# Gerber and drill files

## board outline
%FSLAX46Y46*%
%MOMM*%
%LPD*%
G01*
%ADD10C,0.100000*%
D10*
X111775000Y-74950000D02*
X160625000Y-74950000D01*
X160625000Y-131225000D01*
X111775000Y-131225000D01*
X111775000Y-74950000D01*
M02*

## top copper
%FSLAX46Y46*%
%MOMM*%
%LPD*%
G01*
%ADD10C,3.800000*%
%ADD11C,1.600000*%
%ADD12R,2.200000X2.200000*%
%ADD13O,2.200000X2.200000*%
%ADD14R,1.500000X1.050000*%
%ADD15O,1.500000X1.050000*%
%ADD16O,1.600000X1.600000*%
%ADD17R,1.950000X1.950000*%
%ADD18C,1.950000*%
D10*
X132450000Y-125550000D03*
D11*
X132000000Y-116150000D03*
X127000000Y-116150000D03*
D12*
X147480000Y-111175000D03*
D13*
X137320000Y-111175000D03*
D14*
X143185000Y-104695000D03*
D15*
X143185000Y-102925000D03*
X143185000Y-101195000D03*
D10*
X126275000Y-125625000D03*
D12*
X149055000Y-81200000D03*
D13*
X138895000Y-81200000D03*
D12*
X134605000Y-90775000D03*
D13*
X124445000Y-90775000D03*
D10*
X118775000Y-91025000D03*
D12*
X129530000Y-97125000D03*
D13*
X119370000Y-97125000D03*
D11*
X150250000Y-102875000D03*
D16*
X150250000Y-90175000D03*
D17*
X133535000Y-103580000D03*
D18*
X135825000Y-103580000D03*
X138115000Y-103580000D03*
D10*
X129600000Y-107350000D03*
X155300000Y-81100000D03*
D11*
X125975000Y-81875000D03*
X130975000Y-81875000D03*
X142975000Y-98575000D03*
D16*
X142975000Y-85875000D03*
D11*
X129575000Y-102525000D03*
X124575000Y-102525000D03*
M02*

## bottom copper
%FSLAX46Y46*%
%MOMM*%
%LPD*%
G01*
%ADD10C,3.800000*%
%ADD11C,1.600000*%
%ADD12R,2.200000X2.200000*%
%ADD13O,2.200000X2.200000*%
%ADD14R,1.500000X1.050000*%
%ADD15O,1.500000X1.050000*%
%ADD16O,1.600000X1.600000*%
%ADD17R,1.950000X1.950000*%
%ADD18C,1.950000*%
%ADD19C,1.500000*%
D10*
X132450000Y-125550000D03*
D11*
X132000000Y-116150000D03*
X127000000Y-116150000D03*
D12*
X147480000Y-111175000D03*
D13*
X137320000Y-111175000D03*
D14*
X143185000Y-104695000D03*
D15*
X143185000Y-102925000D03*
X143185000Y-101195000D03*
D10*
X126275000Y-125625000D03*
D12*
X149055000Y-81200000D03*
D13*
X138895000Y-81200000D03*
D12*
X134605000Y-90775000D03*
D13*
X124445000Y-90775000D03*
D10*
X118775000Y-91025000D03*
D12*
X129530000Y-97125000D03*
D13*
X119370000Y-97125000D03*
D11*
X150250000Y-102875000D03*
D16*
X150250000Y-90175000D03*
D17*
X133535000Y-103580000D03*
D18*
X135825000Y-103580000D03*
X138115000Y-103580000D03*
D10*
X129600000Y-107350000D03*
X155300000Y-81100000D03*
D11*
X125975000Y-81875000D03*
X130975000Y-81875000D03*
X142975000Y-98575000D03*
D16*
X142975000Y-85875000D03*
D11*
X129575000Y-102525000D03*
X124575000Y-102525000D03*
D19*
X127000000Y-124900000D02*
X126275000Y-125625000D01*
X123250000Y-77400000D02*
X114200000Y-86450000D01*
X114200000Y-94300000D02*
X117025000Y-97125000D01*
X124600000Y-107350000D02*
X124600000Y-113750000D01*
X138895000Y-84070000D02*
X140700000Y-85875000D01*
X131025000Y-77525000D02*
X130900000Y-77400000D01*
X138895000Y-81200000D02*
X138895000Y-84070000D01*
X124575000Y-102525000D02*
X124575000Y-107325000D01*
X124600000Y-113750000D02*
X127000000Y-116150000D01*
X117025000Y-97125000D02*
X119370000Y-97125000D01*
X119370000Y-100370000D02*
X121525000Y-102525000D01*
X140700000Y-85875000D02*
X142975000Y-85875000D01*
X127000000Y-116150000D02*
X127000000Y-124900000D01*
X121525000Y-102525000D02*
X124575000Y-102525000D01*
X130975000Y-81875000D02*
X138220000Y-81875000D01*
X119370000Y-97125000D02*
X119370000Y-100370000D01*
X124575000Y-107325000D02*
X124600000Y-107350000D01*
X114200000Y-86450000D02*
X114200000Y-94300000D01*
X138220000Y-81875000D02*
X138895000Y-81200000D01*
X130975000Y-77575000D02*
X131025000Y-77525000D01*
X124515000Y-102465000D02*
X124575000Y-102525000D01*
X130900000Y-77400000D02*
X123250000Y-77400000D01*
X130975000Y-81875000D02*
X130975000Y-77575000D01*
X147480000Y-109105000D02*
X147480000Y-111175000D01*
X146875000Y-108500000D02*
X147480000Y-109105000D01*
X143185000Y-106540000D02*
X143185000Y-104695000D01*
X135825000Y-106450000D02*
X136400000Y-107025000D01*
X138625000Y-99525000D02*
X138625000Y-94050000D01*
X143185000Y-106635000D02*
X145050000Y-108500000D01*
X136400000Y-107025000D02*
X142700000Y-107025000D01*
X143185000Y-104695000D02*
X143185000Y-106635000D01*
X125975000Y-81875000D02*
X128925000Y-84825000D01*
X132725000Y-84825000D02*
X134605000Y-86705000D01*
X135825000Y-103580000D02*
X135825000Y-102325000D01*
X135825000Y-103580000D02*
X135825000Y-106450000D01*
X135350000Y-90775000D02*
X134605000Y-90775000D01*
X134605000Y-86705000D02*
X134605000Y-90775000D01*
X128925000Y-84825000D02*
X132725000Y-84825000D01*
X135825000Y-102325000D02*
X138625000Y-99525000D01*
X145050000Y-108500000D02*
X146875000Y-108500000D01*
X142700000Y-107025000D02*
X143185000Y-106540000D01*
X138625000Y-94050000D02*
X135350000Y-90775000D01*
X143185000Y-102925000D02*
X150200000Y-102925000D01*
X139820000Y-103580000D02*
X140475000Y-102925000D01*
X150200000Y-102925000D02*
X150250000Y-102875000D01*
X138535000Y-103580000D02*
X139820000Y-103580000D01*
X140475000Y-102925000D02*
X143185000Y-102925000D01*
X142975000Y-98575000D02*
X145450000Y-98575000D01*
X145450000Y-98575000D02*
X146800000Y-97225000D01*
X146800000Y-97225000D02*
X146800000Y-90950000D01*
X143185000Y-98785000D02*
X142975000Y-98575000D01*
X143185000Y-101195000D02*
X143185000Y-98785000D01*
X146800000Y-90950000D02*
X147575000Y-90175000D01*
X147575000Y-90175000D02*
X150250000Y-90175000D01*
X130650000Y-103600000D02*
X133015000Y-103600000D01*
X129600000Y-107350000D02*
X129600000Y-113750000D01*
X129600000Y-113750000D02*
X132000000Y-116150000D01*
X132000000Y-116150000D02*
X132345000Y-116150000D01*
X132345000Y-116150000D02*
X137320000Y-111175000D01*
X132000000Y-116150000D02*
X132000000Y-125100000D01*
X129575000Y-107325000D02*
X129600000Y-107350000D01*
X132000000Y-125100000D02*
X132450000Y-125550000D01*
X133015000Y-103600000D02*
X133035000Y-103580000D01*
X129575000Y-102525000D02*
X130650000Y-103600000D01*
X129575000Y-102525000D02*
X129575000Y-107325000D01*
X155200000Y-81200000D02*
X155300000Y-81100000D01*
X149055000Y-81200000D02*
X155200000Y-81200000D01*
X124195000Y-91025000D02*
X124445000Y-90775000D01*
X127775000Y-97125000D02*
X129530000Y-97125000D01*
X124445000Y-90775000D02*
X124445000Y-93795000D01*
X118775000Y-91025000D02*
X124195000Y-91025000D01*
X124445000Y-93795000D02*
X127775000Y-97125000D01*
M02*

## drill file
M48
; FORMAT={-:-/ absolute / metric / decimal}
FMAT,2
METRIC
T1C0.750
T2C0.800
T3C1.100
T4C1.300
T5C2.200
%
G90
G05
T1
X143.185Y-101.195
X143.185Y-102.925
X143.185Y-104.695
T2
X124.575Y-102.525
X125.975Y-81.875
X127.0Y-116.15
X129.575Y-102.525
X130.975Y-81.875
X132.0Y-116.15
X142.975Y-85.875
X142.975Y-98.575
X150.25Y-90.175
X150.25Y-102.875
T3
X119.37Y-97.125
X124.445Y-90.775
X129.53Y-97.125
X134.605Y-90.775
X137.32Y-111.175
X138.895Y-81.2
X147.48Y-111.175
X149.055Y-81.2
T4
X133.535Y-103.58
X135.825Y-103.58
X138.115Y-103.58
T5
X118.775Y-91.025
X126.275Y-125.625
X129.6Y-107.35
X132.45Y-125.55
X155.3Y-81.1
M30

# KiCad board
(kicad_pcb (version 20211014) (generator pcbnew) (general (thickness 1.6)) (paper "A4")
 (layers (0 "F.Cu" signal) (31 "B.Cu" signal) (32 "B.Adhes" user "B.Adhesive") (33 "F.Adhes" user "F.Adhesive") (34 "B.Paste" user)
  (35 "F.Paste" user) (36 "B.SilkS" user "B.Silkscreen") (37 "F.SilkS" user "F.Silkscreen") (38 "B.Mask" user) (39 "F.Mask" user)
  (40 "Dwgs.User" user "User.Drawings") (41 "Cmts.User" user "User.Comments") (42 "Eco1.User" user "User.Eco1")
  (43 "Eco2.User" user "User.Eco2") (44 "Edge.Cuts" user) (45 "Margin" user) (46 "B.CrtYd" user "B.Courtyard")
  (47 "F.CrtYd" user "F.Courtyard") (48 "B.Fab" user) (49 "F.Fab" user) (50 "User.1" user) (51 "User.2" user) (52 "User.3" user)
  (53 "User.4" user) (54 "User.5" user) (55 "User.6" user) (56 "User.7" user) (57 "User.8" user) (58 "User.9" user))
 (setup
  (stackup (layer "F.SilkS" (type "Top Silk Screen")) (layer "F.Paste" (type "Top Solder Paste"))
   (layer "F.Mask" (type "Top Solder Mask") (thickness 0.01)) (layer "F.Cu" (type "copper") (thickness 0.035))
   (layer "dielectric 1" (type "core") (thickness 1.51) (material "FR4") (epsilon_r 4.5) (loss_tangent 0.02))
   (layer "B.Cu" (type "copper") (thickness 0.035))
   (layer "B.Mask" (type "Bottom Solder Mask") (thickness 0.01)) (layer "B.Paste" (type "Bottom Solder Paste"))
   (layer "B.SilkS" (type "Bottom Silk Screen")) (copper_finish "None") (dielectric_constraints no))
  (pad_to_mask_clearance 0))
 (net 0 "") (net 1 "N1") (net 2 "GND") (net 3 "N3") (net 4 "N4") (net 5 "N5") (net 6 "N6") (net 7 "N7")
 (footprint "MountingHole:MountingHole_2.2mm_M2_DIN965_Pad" (layer "F.Cu") (at 132.45 125.55)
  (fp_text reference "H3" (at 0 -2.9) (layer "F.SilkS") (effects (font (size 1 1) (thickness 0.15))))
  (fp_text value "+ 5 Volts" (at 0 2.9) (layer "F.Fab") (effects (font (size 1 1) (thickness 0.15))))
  (pad "1" thru_hole circle (at 0 0) (size 3.8 3.8) (drill 2.2) (layers *.Cu *.Mask) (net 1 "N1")))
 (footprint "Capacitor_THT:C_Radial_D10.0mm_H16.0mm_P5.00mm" (layer "F.Cu") (at 132 116.15 180)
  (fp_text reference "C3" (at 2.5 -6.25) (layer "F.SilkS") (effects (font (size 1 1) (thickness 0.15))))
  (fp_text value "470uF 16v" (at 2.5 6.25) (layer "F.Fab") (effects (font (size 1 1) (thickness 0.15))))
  (pad "1" thru_hole circle (at 0 0 180) (size 1.6 1.6) (drill 0.8) (layers *.Cu *.Mask) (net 1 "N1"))
  (pad "2" thru_hole circle (at 5 0 180) (size 1.6 1.6) (drill 0.8) (layers *.Cu *.Mask) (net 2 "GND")))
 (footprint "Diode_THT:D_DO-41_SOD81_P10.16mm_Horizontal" (layer "F.Cu") (at 147.48 111.175 180)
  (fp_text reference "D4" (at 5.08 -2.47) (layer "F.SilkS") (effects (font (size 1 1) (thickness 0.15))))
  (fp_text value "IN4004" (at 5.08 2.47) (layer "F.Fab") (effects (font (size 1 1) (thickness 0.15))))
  (pad "1" thru_hole rect (at 0 0 180) (size 2.2 2.2) (drill 1.1) (layers *.Cu *.Mask) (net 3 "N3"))
  (pad "2" thru_hole oval (at 10.16 0 180) (size 2.2 2.2) (drill 1.1) (layers *.Cu *.Mask) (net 1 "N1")))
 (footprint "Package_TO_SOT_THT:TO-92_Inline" (layer "F.Cu") (at 143.185 104.195 90)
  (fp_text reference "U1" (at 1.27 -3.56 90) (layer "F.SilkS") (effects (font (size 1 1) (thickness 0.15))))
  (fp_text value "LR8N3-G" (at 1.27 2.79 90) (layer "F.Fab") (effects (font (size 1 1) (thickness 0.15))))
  (pad "1" thru_hole rect (at -0.5 0 90) (size 1.05 1.5) (drill 0.75) (layers *.Cu *.Mask) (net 3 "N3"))
  (pad "2" thru_hole oval (at 1.27 0 90) (size 1.05 1.5) (drill 0.75) (layers *.Cu *.Mask) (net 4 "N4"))
  (pad "3" thru_hole oval (at 3 0 90) (size 1.05 1.5) (drill 0.75) (layers *.Cu *.Mask) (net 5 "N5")))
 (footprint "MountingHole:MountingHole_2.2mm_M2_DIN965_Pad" (layer "F.Cu") (at 126.275 125.625)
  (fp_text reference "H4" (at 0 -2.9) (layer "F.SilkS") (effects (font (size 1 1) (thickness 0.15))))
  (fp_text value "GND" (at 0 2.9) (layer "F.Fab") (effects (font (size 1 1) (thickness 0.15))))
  (pad "1" thru_hole circle (at 0 0) (size 3.8 3.8) (drill 2.2) (layers *.Cu *.Mask) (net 2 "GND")))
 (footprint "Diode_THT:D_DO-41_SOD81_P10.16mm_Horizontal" (layer "F.Cu") (at 149.055 81.2 180)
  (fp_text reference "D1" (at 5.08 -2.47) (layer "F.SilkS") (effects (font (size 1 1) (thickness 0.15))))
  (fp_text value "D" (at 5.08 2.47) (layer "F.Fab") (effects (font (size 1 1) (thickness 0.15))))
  (pad "1" thru_hole rect (at 0 0 180) (size 2.2 2.2) (drill 1.1) (layers *.Cu *.Mask) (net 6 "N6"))
  (pad "2" thru_hole oval (at 10.16 0 180) (size 2.2 2.2) (drill 1.1) (layers *.Cu *.Mask) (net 2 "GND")))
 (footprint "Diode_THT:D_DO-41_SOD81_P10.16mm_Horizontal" (layer "F.Cu") (at 134.605 90.775 180)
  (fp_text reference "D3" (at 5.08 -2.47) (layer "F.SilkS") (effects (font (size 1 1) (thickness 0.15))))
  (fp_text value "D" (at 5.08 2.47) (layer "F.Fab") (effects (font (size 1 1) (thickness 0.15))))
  (pad "1" thru_hole rect (at 0 0 180) (size 2.2 2.2) (drill 1.1) (layers *.Cu *.Mask) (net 3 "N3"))
  (pad "2" thru_hole oval (at 10.16 0 180) (size 2.2 2.2) (drill 1.1) (layers *.Cu *.Mask) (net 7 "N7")))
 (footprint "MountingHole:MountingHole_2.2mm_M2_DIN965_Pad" (layer "F.Cu") (at 118.775 91.025)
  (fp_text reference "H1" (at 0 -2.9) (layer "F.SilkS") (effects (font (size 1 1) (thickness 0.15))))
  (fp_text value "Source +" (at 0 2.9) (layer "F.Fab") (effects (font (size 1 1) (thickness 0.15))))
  (pad "1" thru_hole circle (at 0 0) (size 3.8 3.8) (drill 2.2) (layers *.Cu *.Mask) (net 7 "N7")))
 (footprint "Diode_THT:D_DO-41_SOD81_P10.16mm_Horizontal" (layer "F.Cu") (at 129.53 97.125 180)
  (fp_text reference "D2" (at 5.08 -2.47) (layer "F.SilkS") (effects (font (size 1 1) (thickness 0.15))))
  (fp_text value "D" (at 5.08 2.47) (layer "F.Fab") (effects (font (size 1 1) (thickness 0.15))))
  (pad "1" thru_hole rect (at 0 0 180) (size 2.2 2.2) (drill 1.1) (layers *.Cu *.Mask) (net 7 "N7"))
  (pad "2" thru_hole oval (at 10.16 0 180) (size 2.2 2.2) (drill 1.1) (layers *.Cu *.Mask) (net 2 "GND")))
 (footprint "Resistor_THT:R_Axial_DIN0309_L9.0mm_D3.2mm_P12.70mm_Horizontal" (layer "F.Cu") (at 150.25 102.875 90)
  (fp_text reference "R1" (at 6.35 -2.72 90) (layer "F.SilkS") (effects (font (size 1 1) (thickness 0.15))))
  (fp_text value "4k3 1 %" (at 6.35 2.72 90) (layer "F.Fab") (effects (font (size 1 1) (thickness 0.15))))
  (pad "1" thru_hole circle (at 0 0 90) (size 1.6 1.6) (drill 0.8) (layers *.Cu *.Mask) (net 4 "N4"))
  (pad "2" thru_hole oval (at 12.7 0 90) (size 1.6 1.6) (drill 0.8) (layers *.Cu *.Mask) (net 5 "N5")))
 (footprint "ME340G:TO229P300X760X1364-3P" (layer "F.Cu") (at 133.535 103.58)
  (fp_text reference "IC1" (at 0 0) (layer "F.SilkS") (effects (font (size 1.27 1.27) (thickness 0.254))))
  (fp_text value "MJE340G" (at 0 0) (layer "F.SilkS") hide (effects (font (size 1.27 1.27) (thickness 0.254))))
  (pad "1" thru_hole rect locked (at 0 0) (size 1.95 1.95) (drill 1.3) (layers *.Cu *.Mask) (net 1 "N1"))
  (pad "2" thru_hole circle locked (at 2.29 0) (size 1.95 1.95) (drill 1.3) (layers *.Cu *.Mask) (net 3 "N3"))
  (pad "3" thru_hole circle locked (at 4.58 0) (size 1.95 1.95) (drill 1.3) (layers *.Cu *.Mask) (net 4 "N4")))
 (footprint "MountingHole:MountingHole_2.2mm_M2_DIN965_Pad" (layer "F.Cu") (at 129.6 107.35 180)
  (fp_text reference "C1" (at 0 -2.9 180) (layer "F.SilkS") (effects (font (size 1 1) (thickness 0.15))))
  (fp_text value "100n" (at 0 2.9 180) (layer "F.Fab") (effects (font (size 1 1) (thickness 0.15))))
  (pad "1" thru_hole circle (at 0 0 180) (size 3.8 3.8) (drill 2.2) (layers *.Cu *.Mask) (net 1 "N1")))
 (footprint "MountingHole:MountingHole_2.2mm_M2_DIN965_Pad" (layer "F.Cu") (at 155.3 81.1)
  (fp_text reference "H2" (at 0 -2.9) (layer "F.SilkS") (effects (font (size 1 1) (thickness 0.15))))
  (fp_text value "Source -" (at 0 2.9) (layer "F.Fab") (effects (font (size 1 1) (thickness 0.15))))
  (pad "1" thru_hole circle (at 0 0) (size 3.8 3.8) (drill 2.2) (layers *.Cu *.Mask) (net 6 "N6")))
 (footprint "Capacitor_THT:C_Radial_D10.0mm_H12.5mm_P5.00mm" (layer "F.Cu") (at 125.975 81.875)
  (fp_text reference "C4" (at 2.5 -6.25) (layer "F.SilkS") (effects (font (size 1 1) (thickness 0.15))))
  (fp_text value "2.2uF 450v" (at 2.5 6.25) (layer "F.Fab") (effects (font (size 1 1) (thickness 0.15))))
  (pad "1" thru_hole circle (at 0 0) (size 1.6 1.6) (drill 0.8) (layers *.Cu *.Mask) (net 3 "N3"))
  (pad "2" thru_hole circle (at 5 0) (size 1.6 1.6) (drill 0.8) (layers *.Cu *.Mask) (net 2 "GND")))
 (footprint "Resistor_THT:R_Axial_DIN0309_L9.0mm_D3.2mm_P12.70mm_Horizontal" (layer "F.Cu") (at 142.975 98.575 90)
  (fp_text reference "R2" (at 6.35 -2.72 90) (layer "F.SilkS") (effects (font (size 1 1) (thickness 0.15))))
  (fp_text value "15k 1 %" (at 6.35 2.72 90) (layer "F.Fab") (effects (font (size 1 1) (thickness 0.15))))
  (pad "1" thru_hole circle (at 0 0 90) (size 1.6 1.6) (drill 0.8) (layers *.Cu *.Mask) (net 5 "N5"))
  (pad "2" thru_hole oval (at 12.7 0 90) (size 1.6 1.6) (drill 0.8) (layers *.Cu *.Mask) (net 2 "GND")))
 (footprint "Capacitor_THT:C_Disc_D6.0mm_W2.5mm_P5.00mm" (layer "F.Cu") (at 129.575 102.525 180)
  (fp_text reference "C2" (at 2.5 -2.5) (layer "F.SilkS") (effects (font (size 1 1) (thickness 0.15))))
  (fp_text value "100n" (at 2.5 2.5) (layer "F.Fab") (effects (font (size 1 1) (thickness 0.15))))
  (pad "1" thru_hole circle (at 0 0 180) (size 1.6 1.6) (drill 0.8) (layers *.Cu *.Mask) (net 1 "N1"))
  (pad "2" thru_hole circle (at 5 0 180) (size 1.6 1.6) (drill 0.8) (layers *.Cu *.Mask) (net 2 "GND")))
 (gr_rect (start 111.775 74.95) (end 160.625 131.225) (layer "Edge.Cuts") (width 0.1) (fill none))
 (segment (start 127 124.9) (end 126.275 125.625) (width 1.5) (layer "B.Cu") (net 2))
 (segment (start 123.25 77.4) (end 114.2 86.45) (width 1.5) (layer "B.Cu") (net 2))
 (segment (start 114.2 94.3) (end 117.025 97.125) (width 1.5) (layer "B.Cu") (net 2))
 (segment (start 124.6 107.35) (end 124.6 113.75) (width 1.5) (layer "B.Cu") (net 2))
 (segment (start 138.895 84.07) (end 140.7 85.875) (width 1.5) (layer "B.Cu") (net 2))
 (segment (start 131.025 77.525) (end 130.9 77.4) (width 1.5) (layer "B.Cu") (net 2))
 (segment (start 138.895 81.2) (end 138.895 84.07) (width 1.5) (layer "B.Cu") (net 2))
 (segment (start 124.575 102.525) (end 124.575 107.325) (width 1.5) (layer "B.Cu") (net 2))
 (segment (start 124.6 113.75) (end 127 116.15) (width 1.5) (layer "B.Cu") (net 2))
 (segment (start 117.025 97.125) (end 119.37 97.125) (width 1.5) (layer "B.Cu") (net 2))
 (segment (start 119.37 100.37) (end 121.525 102.525) (width 1.5) (layer "B.Cu") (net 2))
 (segment (start 140.7 85.875) (end 142.975 85.875) (width 1.5) (layer "B.Cu") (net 2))
 (segment (start 127 116.15) (end 127 124.9) (width 1.5) (layer "B.Cu") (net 2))
 (segment (start 121.525 102.525) (end 124.575 102.525) (width 1.5) (layer "B.Cu") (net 2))
 (segment (start 130.975 81.875) (end 138.22 81.875) (width 1.5) (layer "B.Cu") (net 2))
 (segment (start 119.37 97.125) (end 119.37 100.37) (width 1.5) (layer "B.Cu") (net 2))
 (segment (start 124.575 107.325) (end 124.6 107.35) (width 1.5) (layer "B.Cu") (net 2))
 (segment (start 114.2 86.45) (end 114.2 94.3) (width 1.5) (layer "B.Cu") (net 2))
 (segment (start 138.22 81.875) (end 138.895 81.2) (width 1.5) (layer "B.Cu") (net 2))
 (segment (start 130.975 77.575) (end 131.025 77.525) (width 1.5) (layer "B.Cu") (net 2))
 (segment (start 124.515 102.465) (end 124.575 102.525) (width 1.5) (layer "B.Cu") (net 2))
 (segment (start 130.9 77.4) (end 123.25 77.4) (width 1.5) (layer "B.Cu") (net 2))
 (segment (start 130.975 81.875) (end 130.975 77.575) (width 1.5) (layer "B.Cu") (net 2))
 (segment (start 147.48 109.105) (end 147.48 111.175) (width 1.5) (layer "B.Cu") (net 3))
 (segment (start 146.875 108.5) (end 147.48 109.105) (width 1.5) (layer "B.Cu") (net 3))
 (segment (start 143.185 106.54) (end 143.185 104.695) (width 1.5) (layer "B.Cu") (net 3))
 (segment (start 135.825 106.45) (end 136.4 107.025) (width 1.5) (layer "B.Cu") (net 3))
 (segment (start 138.625 99.525) (end 138.625 94.05) (width 1.5) (layer "B.Cu") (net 3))
 (segment (start 143.185 106.635) (end 145.05 108.5) (width 1.5) (layer "B.Cu") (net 3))
 (segment (start 136.4 107.025) (end 142.7 107.025) (width 1.5) (layer "B.Cu") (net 3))
 (segment (start 143.185 104.695) (end 143.185 106.635) (width 1.5) (layer "B.Cu") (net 3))
 (segment (start 125.975 81.875) (end 128.925 84.825) (width 1.5) (layer "B.Cu") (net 3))
 (segment (start 132.725 84.825) (end 134.605 86.705) (width 1.5) (layer "B.Cu") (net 3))
 (segment (start 135.825 103.58) (end 135.825 102.325) (width 1.5) (layer "B.Cu") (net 3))
 (segment (start 135.825 103.58) (end 135.825 106.45) (width 1.5) (layer "B.Cu") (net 3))
 (segment (start 135.35 90.775) (end 134.605 90.775) (width 1.5) (layer "B.Cu") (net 3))
 (segment (start 134.605 86.705) (end 134.605 90.775) (width 1.5) (layer "B.Cu") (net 3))
 (segment (start 128.925 84.825) (end 132.725 84.825) (width 1.5) (layer "B.Cu") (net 3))
 (segment (start 135.825 102.325) (end 138.625 99.525) (width 1.5) (layer "B.Cu") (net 3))
 (segment (start 145.05 108.5) (end 146.875 108.5) (width 1.5) (layer "B.Cu") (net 3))
 (segment (start 142.7 107.025) (end 143.185 106.54) (width 1.5) (layer "B.Cu") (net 3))
 (segment (start 138.625 94.05) (end 135.35 90.775) (width 1.5) (layer "B.Cu") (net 3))
 (segment (start 143.185 102.925) (end 150.2 102.925) (width 1.5) (layer "B.Cu") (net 4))
 (segment (start 139.82 103.58) (end 140.475 102.925) (width 1.5) (layer "B.Cu") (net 4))
 (segment (start 150.2 102.925) (end 150.25 102.875) (width 1.5) (layer "B.Cu") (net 4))
 (segment (start 138.535 103.58) (end 139.82 103.58) (width 1.5) (layer "B.Cu") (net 4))
 (segment (start 140.475 102.925) (end 143.185 102.925) (width 1.5) (layer "B.Cu") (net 4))
 (segment (start 142.975 98.575) (end 145.45 98.575) (width 1.5) (layer "B.Cu") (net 5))
 (segment (start 145.45 98.575) (end 146.8 97.225) (width 1.5) (layer "B.Cu") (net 5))
 (segment (start 146.8 97.225) (end 146.8 90.95) (width 1.5) (layer "B.Cu") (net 5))
 (segment (start 143.185 98.785) (end 142.975 98.575) (width 1.5) (layer "B.Cu") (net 5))
 (segment (start 143.185 101.195) (end 143.185 98.785) (width 1.5) (layer "B.Cu") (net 5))
 (segment (start 146.8 90.95) (end 147.575 90.175) (width 1.5) (layer "B.Cu") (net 5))
 (segment (start 147.575 90.175) (end 150.25 90.175) (width 1.5) (layer "B.Cu") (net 5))
 (segment (start 130.65 103.6) (end 133.015 103.6) (width 1.5) (layer "B.Cu") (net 1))
 (segment (start 129.6 107.35) (end 129.6 113.75) (width 1.5) (layer "B.Cu") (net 1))
 (segment (start 129.6 113.75) (end 132 116.15) (width 1.5) (layer "B.Cu") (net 1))
 (segment (start 132 116.15) (end 132.345 116.15) (width 1.5) (layer "B.Cu") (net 1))
 (segment (start 132.345 116.15) (end 137.32 111.175) (width 1.5) (layer "B.Cu") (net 1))
 (segment (start 132 116.15) (end 132 125.1) (width 1.5) (layer "B.Cu") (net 1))
 (segment (start 129.575 107.325) (end 129.6 107.35) (width 1.5) (layer "B.Cu") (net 1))
 (segment (start 132 125.1) (end 132.45 125.55) (width 1.5) (layer "B.Cu") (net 1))
 (segment (start 133.015 103.6) (end 133.035 103.58) (width 1.5) (layer "B.Cu") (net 1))
 (segment (start 129.575 102.525) (end 130.65 103.6) (width 1.5) (layer "B.Cu") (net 1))
 (segment (start 129.575 102.525) (end 129.575 107.325) (width 1.5) (layer "B.Cu") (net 1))
 (segment (start 155.2 81.2) (end 155.3 81.1) (width 1.5) (layer "B.Cu") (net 6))
 (segment (start 149.055 81.2) (end 155.2 81.2) (width 1.5) (layer "B.Cu") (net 6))
 (segment (start 124.195 91.025) (end 124.445 90.775) (width 1.5) (layer "B.Cu") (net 7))
 (segment (start 127.775 97.125) (end 129.53 97.125) (width 1.5) (layer "B.Cu") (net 7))
 (segment (start 124.445 90.775) (end 124.445 93.795) (width 1.5) (layer "B.Cu") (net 7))
 (segment (start 118.775 91.025) (end 124.195 91.025) (width 1.5) (layer "B.Cu") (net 7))
 (segment (start 124.445 93.795) (end 127.775 97.125) (width 1.5) (layer "B.Cu") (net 7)))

